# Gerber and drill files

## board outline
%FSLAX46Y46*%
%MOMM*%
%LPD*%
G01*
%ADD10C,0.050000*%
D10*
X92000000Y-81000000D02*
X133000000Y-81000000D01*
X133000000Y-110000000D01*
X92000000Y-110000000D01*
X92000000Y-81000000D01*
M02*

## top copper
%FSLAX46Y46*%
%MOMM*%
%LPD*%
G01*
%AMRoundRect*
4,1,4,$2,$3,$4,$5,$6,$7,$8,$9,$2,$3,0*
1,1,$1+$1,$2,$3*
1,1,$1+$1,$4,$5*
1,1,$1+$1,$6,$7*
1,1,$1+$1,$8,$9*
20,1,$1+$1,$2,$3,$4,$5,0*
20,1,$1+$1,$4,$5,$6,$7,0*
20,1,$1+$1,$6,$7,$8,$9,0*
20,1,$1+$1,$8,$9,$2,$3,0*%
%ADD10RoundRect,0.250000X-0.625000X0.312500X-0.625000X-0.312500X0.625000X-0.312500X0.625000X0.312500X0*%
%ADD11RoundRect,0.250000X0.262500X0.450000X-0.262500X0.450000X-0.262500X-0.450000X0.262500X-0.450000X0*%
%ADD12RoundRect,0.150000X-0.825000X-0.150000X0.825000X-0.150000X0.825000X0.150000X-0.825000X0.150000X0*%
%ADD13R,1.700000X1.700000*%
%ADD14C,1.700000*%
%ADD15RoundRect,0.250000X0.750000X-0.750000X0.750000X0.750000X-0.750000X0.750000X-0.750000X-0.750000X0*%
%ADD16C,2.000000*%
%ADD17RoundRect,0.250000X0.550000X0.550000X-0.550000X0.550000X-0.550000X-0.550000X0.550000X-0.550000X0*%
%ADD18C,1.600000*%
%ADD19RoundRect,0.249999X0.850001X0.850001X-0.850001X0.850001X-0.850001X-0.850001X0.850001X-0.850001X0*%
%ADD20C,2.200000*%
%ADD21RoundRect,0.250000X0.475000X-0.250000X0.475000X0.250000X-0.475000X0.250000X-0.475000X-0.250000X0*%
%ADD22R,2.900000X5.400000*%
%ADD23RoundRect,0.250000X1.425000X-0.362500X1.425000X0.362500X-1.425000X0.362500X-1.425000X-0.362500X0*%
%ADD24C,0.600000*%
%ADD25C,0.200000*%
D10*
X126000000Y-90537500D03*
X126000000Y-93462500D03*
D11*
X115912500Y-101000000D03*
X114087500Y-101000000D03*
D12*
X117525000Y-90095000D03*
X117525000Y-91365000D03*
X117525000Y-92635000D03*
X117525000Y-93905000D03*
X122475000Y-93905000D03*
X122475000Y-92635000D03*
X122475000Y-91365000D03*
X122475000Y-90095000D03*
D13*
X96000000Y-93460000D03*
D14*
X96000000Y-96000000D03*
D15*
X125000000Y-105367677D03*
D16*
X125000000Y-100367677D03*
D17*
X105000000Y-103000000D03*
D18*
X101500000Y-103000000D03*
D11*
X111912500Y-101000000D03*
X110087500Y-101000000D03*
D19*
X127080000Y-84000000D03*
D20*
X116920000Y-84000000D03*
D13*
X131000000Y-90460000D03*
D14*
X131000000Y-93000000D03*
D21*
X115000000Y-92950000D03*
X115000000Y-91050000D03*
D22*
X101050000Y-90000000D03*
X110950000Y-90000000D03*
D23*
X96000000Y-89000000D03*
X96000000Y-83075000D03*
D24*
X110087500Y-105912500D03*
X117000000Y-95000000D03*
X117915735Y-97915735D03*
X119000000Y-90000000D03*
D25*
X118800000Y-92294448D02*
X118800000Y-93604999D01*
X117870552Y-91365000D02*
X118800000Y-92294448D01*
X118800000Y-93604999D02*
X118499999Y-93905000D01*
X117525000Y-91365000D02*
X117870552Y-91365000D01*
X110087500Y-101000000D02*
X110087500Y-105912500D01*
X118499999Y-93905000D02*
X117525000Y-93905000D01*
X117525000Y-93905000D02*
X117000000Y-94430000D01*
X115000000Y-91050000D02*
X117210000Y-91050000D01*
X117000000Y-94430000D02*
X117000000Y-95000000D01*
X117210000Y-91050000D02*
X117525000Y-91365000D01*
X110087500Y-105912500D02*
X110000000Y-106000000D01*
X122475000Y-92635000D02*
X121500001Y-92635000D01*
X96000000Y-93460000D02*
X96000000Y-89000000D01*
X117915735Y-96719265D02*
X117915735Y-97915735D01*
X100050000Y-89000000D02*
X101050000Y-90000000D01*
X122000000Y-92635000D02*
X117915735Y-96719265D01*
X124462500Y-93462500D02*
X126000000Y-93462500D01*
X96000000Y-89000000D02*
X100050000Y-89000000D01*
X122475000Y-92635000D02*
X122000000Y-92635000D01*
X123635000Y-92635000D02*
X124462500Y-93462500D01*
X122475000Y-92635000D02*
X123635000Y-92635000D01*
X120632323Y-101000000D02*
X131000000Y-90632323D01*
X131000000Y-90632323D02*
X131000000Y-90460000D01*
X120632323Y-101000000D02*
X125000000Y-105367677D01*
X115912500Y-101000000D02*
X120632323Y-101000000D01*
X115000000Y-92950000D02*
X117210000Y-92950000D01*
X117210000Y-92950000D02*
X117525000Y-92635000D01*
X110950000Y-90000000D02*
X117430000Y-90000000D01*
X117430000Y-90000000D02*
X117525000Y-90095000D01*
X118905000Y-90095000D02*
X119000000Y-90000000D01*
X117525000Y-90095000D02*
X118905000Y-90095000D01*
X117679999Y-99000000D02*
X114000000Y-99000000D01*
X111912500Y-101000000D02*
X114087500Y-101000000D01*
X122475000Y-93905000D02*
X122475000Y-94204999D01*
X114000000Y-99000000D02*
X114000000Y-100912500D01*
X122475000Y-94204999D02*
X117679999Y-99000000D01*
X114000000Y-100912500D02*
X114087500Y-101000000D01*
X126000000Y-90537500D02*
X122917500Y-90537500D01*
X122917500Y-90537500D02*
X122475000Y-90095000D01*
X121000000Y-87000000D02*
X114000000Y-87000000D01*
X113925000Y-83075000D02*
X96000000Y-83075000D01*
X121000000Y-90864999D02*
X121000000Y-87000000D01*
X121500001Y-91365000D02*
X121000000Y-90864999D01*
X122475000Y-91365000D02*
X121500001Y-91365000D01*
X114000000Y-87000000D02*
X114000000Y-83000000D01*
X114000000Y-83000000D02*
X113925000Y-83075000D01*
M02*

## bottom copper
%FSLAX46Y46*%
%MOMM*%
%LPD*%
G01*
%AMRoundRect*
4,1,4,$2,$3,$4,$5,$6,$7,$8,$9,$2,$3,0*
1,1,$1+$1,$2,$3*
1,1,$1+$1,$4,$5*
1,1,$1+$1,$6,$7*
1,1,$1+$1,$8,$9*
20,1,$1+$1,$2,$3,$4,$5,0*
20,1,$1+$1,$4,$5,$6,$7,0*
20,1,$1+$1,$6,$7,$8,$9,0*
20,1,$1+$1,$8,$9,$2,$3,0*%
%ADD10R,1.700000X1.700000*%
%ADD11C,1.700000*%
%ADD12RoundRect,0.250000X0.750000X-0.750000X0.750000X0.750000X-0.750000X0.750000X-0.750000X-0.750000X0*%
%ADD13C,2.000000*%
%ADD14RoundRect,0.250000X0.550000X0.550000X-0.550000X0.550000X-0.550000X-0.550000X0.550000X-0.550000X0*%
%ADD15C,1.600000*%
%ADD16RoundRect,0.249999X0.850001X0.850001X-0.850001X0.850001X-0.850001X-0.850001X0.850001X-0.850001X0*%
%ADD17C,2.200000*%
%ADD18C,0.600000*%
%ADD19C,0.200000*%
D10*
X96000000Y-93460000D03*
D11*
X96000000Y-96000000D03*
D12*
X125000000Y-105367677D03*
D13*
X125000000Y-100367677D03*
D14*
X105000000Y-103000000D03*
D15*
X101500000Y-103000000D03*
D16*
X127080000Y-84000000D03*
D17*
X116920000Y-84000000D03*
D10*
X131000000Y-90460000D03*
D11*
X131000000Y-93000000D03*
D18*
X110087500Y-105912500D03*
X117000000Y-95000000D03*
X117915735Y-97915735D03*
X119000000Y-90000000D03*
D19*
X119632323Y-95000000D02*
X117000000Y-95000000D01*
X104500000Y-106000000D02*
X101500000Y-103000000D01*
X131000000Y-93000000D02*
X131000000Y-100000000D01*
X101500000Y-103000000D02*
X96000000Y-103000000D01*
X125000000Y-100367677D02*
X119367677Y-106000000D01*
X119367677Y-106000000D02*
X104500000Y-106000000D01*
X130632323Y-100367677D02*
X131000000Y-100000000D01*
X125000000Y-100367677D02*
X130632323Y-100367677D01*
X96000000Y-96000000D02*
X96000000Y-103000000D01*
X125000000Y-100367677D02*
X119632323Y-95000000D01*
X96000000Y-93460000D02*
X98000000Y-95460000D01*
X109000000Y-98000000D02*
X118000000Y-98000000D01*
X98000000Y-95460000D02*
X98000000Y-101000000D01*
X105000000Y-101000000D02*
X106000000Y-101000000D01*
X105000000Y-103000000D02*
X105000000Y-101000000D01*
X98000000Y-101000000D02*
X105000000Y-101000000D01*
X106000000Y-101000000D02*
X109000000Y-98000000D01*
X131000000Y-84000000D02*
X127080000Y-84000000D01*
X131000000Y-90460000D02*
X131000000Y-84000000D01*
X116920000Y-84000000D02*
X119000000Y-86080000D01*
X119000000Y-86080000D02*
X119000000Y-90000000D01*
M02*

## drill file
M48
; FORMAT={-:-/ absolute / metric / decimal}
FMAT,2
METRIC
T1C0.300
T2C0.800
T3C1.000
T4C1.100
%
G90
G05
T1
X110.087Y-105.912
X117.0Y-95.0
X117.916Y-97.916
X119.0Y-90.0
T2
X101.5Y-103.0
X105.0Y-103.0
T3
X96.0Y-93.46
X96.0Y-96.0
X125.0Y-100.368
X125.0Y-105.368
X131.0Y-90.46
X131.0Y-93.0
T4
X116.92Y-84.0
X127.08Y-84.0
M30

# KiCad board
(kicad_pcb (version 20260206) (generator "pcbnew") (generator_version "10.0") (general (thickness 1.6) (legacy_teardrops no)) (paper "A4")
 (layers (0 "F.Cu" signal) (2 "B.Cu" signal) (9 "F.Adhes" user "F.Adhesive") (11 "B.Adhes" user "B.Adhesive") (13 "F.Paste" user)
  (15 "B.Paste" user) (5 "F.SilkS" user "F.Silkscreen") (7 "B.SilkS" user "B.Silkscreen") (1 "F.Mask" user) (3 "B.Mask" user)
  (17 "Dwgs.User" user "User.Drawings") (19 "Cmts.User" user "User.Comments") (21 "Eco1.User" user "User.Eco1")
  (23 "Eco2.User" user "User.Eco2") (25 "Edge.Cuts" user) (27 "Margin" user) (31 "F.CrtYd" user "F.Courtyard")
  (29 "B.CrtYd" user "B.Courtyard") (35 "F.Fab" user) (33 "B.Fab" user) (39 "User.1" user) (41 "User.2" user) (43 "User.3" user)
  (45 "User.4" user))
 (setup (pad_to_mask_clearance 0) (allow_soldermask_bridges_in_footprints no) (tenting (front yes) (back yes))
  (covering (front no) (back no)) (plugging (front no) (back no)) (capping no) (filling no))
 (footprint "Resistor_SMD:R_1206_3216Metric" (layer "F.Cu") (at 126 92 -90)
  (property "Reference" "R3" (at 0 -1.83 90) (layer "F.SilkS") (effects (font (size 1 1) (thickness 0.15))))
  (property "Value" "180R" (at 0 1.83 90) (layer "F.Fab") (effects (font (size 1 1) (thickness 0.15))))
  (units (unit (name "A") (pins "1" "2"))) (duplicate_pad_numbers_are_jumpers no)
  (pad "1" smd roundrect (at -1.4625 0 270) (size 1.125 1.75) (layers "F.Cu" "F.Mask" "F.Paste") (roundrect_rratio 0.222222) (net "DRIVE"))
  (pad "2" smd roundrect (at 1.4625 0 270) (size 1.125 1.75) (layers "F.Cu" "F.Mask" "F.Paste") (roundrect_rratio 0.222222) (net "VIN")))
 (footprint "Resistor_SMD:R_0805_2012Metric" (layer "F.Cu") (at 115 101 180)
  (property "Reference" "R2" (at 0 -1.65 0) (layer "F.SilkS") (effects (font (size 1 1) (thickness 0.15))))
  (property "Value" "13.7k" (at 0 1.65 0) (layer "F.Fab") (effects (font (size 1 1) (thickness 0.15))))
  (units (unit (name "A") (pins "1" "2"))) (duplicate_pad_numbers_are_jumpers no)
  (pad "1" smd roundrect (at -0.9125 0 180) (size 1.025 1.4) (layers "F.Cu" "F.Mask" "F.Paste") (roundrect_rratio 0.243902) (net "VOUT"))
  (pad "2" smd roundrect (at 0.9125 0 180) (size 1.025 1.4) (layers "F.Cu" "F.Mask" "F.Paste") (roundrect_rratio 0.243902) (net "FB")))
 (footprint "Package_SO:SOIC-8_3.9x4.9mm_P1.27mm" (layer "F.Cu") (at 120 92)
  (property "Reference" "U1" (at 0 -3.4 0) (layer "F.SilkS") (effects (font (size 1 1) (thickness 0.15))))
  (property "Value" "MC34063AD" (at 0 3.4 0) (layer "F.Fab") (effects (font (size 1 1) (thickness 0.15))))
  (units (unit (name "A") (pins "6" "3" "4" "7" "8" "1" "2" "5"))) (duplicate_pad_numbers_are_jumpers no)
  (pad "1" smd roundrect (at -2.475 -1.905) (size 1.95 0.6) (layers "F.Cu" "F.Mask" "F.Paste") (roundrect_rratio 0.25) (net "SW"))
  (pad "2" smd roundrect (at -2.475 -0.635) (size 1.95 0.6) (layers "F.Cu" "F.Mask" "F.Paste") (roundrect_rratio 0.25) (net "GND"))
  (pad "3" smd roundrect (at -2.475 0.635) (size 1.95 0.6) (layers "F.Cu" "F.Mask" "F.Paste") (roundrect_rratio 0.25) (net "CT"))
  (pad "4" smd roundrect (at -2.475 1.905) (size 1.95 0.6) (layers "F.Cu" "F.Mask" "F.Paste") (roundrect_rratio 0.25) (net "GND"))
  (pad "5" smd roundrect (at 2.475 1.905) (size 1.95 0.6) (layers "F.Cu" "F.Mask" "F.Paste") (roundrect_rratio 0.25) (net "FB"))
  (pad "6" smd roundrect (at 2.475 0.635) (size 1.95 0.6) (layers "F.Cu" "F.Mask" "F.Paste") (roundrect_rratio 0.25) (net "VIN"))
  (pad "7" smd roundrect (at 2.475 -0.635) (size 1.95 0.6) (layers "F.Cu" "F.Mask" "F.Paste") (roundrect_rratio 0.25) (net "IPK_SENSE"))
  (pad "8" smd roundrect (at 2.475 -1.905) (size 1.95 0.6) (layers "F.Cu" "F.Mask" "F.Paste") (roundrect_rratio 0.25) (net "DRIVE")))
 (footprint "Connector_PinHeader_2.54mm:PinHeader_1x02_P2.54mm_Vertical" (layer "F.Cu") (at 96 93.46)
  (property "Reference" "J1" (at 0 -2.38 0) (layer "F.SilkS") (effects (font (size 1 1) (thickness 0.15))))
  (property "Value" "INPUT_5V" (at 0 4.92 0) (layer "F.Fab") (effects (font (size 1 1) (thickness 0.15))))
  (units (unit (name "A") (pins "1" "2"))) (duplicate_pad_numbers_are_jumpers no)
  (pad "1" thru_hole rect (at 0 0) (size 1.7 1.7) (drill 1) (layers "*.Cu" "*.Mask") (remove_unused_layers no) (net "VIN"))
  (pad "2" thru_hole circle (at 0 2.54) (size 1.7 1.7) (drill 1) (layers "*.Cu" "*.Mask") (remove_unused_layers no) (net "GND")))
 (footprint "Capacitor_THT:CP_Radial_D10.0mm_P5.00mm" (layer "F.Cu") (at 125 105.367677 90)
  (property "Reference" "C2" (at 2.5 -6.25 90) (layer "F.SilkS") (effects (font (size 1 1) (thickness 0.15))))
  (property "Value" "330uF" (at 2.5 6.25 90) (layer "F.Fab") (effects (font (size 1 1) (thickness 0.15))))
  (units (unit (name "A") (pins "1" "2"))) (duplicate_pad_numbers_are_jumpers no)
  (pad "1" thru_hole roundrect (at 0 0 90) (size 2 2) (drill 1) (layers "*.Cu" "*.Mask") (remove_unused_layers no) (roundrect_rratio 0.125)
   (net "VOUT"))
  (pad "2" thru_hole circle (at 5 0 90) (size 2 2) (drill 1) (layers "*.Cu" "*.Mask") (remove_unused_layers no) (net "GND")))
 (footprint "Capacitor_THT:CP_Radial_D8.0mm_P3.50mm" (layer "F.Cu") (at 105 103 180)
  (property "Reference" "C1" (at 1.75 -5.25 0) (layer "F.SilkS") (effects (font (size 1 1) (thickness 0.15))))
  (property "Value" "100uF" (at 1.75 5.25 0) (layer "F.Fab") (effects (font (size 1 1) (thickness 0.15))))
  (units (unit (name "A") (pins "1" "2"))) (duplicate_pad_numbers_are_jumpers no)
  (pad "1" thru_hole roundrect (at 0 0 180) (size 1.6 1.6) (drill 0.8) (layers "*.Cu" "*.Mask") (remove_unused_layers no)
   (roundrect_rratio 0.15625) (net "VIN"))
  (pad "2" thru_hole circle (at 3.5 0 180) (size 1.6 1.6) (drill 0.8) (layers "*.Cu" "*.Mask") (remove_unused_layers no) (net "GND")))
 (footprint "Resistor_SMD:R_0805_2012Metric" (layer "F.Cu") (at 111 101 180)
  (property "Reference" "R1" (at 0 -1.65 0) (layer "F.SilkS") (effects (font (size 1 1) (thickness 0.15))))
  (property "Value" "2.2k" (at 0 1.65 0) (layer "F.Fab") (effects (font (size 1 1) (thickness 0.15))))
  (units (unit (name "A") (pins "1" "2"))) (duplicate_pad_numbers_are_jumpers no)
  (pad "1" smd roundrect (at -0.9125 0 180) (size 1.025 1.4) (layers "F.Cu" "F.Mask" "F.Paste") (roundrect_rratio 0.243902) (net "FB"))
  (pad "2" smd roundrect (at 0.9125 0 180) (size 1.025 1.4) (layers "F.Cu" "F.Mask" "F.Paste") (roundrect_rratio 0.243902) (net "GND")))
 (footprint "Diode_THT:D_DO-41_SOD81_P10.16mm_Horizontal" (layer "F.Cu") (at 127.08 84 180)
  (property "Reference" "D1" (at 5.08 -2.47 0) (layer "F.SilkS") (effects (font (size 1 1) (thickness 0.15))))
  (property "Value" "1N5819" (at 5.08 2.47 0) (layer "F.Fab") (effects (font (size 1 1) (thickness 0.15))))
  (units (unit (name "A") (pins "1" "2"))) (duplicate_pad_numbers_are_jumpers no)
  (pad "1" thru_hole roundrect (at 0 0 180) (size 2.2 2.2) (drill 1.1) (layers "*.Cu" "*.Mask") (remove_unused_layers no)
   (roundrect_rratio 0.113636) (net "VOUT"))
  (pad "2" thru_hole circle (at 10.16 0 180) (size 2.2 2.2) (drill 1.1) (layers "*.Cu" "*.Mask") (remove_unused_layers no) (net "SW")))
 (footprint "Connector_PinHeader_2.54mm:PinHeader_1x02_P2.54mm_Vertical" (layer "F.Cu") (at 131 90.46)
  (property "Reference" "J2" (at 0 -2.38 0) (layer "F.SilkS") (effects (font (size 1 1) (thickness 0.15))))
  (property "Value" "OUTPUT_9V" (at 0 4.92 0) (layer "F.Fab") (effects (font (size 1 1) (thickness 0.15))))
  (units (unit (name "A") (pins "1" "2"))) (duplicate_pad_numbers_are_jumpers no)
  (pad "1" thru_hole rect (at 0 0) (size 1.7 1.7) (drill 1) (layers "*.Cu" "*.Mask") (remove_unused_layers no) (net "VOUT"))
  (pad "2" thru_hole circle (at 0 2.54) (size 1.7 1.7) (drill 1) (layers "*.Cu" "*.Mask") (remove_unused_layers no) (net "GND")))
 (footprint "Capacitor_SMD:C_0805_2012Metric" (layer "F.Cu") (at 115 92 90)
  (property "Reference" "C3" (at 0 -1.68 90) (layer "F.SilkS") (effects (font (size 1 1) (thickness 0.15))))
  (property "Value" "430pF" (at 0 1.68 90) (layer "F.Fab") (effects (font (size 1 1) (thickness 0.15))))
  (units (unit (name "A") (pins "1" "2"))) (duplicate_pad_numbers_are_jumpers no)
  (pad "1" smd roundrect (at -0.95 0 90) (size 1 1.45) (layers "F.Cu" "F.Mask" "F.Paste") (roundrect_rratio 0.25) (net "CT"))
  (pad "2" smd roundrect (at 0.95 0 90) (size 1 1.45) (layers "F.Cu" "F.Mask" "F.Paste") (roundrect_rratio 0.25) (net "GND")))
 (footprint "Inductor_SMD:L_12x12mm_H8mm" (layer "F.Cu") (at 106 90)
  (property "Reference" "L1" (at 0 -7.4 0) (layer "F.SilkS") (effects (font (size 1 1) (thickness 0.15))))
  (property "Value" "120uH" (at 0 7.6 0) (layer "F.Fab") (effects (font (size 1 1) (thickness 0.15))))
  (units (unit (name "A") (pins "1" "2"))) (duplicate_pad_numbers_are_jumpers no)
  (pad "1" smd rect (at -4.95 0) (size 2.9 5.4) (layers "F.Cu" "F.Mask" "F.Paste") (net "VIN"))
  (pad "2" smd rect (at 4.95 0) (size 2.9 5.4) (layers "F.Cu" "F.Mask" "F.Paste") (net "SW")))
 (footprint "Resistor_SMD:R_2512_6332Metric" (layer "F.Cu") (at 96 86.0375 90)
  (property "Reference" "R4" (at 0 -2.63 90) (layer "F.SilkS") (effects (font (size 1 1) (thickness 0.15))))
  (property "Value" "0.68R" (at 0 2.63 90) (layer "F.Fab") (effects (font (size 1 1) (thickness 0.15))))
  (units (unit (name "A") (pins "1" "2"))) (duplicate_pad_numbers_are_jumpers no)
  (pad "1" smd roundrect (at -2.9625 0 90) (size 1.225 3.35) (layers "F.Cu" "F.Mask" "F.Paste") (roundrect_rratio 0.204082) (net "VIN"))
  (pad "2" smd roundrect (at 2.9625 0 90) (size 1.225 3.35) (layers "F.Cu" "F.Mask" "F.Paste") (roundrect_rratio 0.204082) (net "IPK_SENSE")))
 (gr_rect (start 92 81) (end 133 110) (stroke (width 0.05) (type default)) (fill no) (layer "Edge.Cuts"))
 (segment (start 118.8 92.294448) (end 118.8 93.604999) (width 0.2) (layer "F.Cu") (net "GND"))
 (segment (start 117.870552 91.365) (end 118.8 92.294448) (width 0.2) (layer "F.Cu") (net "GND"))
 (segment (start 118.8 93.604999) (end 118.499999 93.905) (width 0.2) (layer "F.Cu") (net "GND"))
 (segment (start 117.525 91.365) (end 117.870552 91.365) (width 0.2) (layer "F.Cu") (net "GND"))
 (segment (start 110.0875 101) (end 110.0875 105.9125) (width 0.2) (layer "F.Cu") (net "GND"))
 (segment (start 118.499999 93.905) (end 117.525 93.905) (width 0.2) (layer "F.Cu") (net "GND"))
 (segment (start 117.525 93.905) (end 117 94.43) (width 0.2) (layer "F.Cu") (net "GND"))
 (segment (start 115 91.05) (end 117.21 91.05) (width 0.2) (layer "F.Cu") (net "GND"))
 (segment (start 117 94.43) (end 117 95) (width 0.2) (layer "F.Cu") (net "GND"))
 (segment (start 117.21 91.05) (end 117.525 91.365) (width 0.2) (layer "F.Cu") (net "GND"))
 (segment (start 110.0875 105.9125) (end 110 106) (width 0.2) (layer "F.Cu") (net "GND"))
 (via (at 110.0875 105.9125) (size 0.6) (drill 0.3) (layers "F.Cu" "B.Cu") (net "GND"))
 (via (at 117 95) (size 0.6) (drill 0.3) (layers "F.Cu" "B.Cu") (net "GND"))
 (segment (start 119.632323 95) (end 117 95) (width 0.2) (layer "B.Cu") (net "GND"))
 (segment (start 104.5 106) (end 101.5 103) (width 0.2) (layer "B.Cu") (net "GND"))
 (segment (start 131 93) (end 131 100) (width 0.2) (layer "B.Cu") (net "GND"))
 (segment (start 101.5 103) (end 96 103) (width 0.2) (layer "B.Cu") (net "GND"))
 (segment (start 125 100.367677) (end 119.367677 106) (width 0.2) (layer "B.Cu") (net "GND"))
 (segment (start 119.367677 106) (end 104.5 106) (width 0.2) (layer "B.Cu") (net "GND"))
 (segment (start 130.632323 100.367677) (end 131 100) (width 0.2) (layer "B.Cu") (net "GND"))
 (segment (start 125 100.367677) (end 130.632323 100.367677) (width 0.2) (layer "B.Cu") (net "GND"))
 (segment (start 96 96) (end 96 103) (width 0.2) (layer "B.Cu") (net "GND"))
 (segment (start 125 100.367677) (end 119.632323 95) (width 0.2) (layer "B.Cu") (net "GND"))
 (segment (start 122.475 92.635) (end 121.500001 92.635) (width 0.2) (layer "F.Cu") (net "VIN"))
 (segment (start 96 93.46) (end 96 89) (width 0.2) (layer "F.Cu") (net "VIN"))
 (segment (start 117.915735 96.719265) (end 117.915735 97.915735) (width 0.2) (layer "F.Cu") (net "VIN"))
 (segment (start 100.05 89) (end 101.05 90) (width 0.2) (layer "F.Cu") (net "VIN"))
 (segment (start 122 92.635) (end 117.915735 96.719265) (width 0.2) (layer "F.Cu") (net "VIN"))
 (segment (start 124.4625 93.4625) (end 126 93.4625) (width 0.2) (layer "F.Cu") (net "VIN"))
 (segment (start 96 89) (end 100.05 89) (width 0.2) (layer "F.Cu") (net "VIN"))
 (segment (start 122.475 92.635) (end 122 92.635) (width 0.2) (layer "F.Cu") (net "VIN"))
 (segment (start 123.635 92.635) (end 124.4625 93.4625) (width 0.2) (layer "F.Cu") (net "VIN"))
 (segment (start 122.475 92.635) (end 123.635 92.635) (width 0.2) (layer "F.Cu") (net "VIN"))
 (via (at 117.915735 97.915735) (size 0.6) (drill 0.3) (layers "F.Cu" "B.Cu") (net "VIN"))
 (segment (start 96 93.46) (end 98 95.46) (width 0.2) (layer "B.Cu") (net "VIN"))
 (segment (start 109 98) (end 118 98) (width 0.2) (layer "B.Cu") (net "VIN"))
 (segment (start 98 95.46) (end 98 101) (width 0.2) (layer "B.Cu") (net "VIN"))
 (segment (start 105 101) (end 106 101) (width 0.2) (layer "B.Cu") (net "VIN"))
 (segment (start 105 103) (end 105 101) (width 0.2) (layer "B.Cu") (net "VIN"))
 (segment (start 98 101) (end 105 101) (width 0.2) (layer "B.Cu") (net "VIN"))
 (segment (start 106 101) (end 109 98) (width 0.2) (layer "B.Cu") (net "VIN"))
 (segment (start 120.632323 101) (end 131 90.632323) (width 0.2) (layer "F.Cu") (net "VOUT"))
 (segment (start 131 90.632323) (end 131 90.46) (width 0.2) (layer "F.Cu") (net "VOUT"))
 (segment (start 120.632323 101) (end 125 105.367677) (width 0.2) (layer "F.Cu") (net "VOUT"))
 (segment (start 115.9125 101) (end 120.632323 101) (width 0.2) (layer "F.Cu") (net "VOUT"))
 (segment (start 131 84) (end 127.08 84) (width 0.2) (layer "B.Cu") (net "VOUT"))
 (segment (start 131 90.46) (end 131 84) (width 0.2) (layer "B.Cu") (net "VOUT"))
 (segment (start 115 92.95) (end 117.21 92.95) (width 0.2) (layer "F.Cu") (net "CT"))
 (segment (start 117.21 92.95) (end 117.525 92.635) (width 0.2) (layer "F.Cu") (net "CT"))
 (segment (start 110.95 90) (end 117.43 90) (width 0.2) (layer "F.Cu") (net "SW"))
 (segment (start 117.43 90) (end 117.525 90.095) (width 0.2) (layer "F.Cu") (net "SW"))
 (segment (start 118.905 90.095) (end 119 90) (width 0.2) (layer "F.Cu") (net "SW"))
 (segment (start 117.525 90.095) (end 118.905 90.095) (width 0.2) (layer "F.Cu") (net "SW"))
 (via (at 119 90) (size 0.6) (drill 0.3) (layers "F.Cu" "B.Cu") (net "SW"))
 (segment (start 116.92 84) (end 119 86.08) (width 0.2) (layer "B.Cu") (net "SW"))
 (segment (start 119 86.08) (end 119 90) (width 0.2) (layer "B.Cu") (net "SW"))
 (segment (start 117.679999 99) (end 114 99) (width 0.2) (layer "F.Cu") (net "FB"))
 (segment (start 111.9125 101) (end 114.0875 101) (width 0.2) (layer "F.Cu") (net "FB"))
 (segment (start 122.475 93.905) (end 122.475 94.204999) (width 0.2) (layer "F.Cu") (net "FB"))
 (segment (start 114 99) (end 114 100.9125) (width 0.2) (layer "F.Cu") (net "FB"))
 (segment (start 122.475 94.204999) (end 117.679999 99) (width 0.2) (layer "F.Cu") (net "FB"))
 (segment (start 114 100.9125) (end 114.0875 101) (width 0.2) (layer "F.Cu") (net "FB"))
 (segment (start 126 90.5375) (end 122.9175 90.5375) (width 0.2) (layer "F.Cu") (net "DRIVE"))
 (segment (start 122.9175 90.5375) (end 122.475 90.095) (width 0.2) (layer "F.Cu") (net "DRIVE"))
 (segment (start 121 87) (end 114 87) (width 0.2) (layer "F.Cu") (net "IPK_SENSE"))
 (segment (start 113.925 83.075) (end 96 83.075) (width 0.2) (layer "F.Cu") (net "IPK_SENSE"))
 (segment (start 121 90.864999) (end 121 87) (width 0.2) (layer "F.Cu") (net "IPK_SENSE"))
 (segment (start 121.500001 91.365) (end 121 90.864999) (width 0.2) (layer "F.Cu") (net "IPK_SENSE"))
 (segment (start 122.475 91.365) (end 121.500001 91.365) (width 0.2) (layer "F.Cu") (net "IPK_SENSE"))
 (segment (start 114 87) (end 114 83) (width 0.2) (layer "F.Cu") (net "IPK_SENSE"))
 (segment (start 114 83) (end 113.925 83.075) (width 0.2) (layer "F.Cu") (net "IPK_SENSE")))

